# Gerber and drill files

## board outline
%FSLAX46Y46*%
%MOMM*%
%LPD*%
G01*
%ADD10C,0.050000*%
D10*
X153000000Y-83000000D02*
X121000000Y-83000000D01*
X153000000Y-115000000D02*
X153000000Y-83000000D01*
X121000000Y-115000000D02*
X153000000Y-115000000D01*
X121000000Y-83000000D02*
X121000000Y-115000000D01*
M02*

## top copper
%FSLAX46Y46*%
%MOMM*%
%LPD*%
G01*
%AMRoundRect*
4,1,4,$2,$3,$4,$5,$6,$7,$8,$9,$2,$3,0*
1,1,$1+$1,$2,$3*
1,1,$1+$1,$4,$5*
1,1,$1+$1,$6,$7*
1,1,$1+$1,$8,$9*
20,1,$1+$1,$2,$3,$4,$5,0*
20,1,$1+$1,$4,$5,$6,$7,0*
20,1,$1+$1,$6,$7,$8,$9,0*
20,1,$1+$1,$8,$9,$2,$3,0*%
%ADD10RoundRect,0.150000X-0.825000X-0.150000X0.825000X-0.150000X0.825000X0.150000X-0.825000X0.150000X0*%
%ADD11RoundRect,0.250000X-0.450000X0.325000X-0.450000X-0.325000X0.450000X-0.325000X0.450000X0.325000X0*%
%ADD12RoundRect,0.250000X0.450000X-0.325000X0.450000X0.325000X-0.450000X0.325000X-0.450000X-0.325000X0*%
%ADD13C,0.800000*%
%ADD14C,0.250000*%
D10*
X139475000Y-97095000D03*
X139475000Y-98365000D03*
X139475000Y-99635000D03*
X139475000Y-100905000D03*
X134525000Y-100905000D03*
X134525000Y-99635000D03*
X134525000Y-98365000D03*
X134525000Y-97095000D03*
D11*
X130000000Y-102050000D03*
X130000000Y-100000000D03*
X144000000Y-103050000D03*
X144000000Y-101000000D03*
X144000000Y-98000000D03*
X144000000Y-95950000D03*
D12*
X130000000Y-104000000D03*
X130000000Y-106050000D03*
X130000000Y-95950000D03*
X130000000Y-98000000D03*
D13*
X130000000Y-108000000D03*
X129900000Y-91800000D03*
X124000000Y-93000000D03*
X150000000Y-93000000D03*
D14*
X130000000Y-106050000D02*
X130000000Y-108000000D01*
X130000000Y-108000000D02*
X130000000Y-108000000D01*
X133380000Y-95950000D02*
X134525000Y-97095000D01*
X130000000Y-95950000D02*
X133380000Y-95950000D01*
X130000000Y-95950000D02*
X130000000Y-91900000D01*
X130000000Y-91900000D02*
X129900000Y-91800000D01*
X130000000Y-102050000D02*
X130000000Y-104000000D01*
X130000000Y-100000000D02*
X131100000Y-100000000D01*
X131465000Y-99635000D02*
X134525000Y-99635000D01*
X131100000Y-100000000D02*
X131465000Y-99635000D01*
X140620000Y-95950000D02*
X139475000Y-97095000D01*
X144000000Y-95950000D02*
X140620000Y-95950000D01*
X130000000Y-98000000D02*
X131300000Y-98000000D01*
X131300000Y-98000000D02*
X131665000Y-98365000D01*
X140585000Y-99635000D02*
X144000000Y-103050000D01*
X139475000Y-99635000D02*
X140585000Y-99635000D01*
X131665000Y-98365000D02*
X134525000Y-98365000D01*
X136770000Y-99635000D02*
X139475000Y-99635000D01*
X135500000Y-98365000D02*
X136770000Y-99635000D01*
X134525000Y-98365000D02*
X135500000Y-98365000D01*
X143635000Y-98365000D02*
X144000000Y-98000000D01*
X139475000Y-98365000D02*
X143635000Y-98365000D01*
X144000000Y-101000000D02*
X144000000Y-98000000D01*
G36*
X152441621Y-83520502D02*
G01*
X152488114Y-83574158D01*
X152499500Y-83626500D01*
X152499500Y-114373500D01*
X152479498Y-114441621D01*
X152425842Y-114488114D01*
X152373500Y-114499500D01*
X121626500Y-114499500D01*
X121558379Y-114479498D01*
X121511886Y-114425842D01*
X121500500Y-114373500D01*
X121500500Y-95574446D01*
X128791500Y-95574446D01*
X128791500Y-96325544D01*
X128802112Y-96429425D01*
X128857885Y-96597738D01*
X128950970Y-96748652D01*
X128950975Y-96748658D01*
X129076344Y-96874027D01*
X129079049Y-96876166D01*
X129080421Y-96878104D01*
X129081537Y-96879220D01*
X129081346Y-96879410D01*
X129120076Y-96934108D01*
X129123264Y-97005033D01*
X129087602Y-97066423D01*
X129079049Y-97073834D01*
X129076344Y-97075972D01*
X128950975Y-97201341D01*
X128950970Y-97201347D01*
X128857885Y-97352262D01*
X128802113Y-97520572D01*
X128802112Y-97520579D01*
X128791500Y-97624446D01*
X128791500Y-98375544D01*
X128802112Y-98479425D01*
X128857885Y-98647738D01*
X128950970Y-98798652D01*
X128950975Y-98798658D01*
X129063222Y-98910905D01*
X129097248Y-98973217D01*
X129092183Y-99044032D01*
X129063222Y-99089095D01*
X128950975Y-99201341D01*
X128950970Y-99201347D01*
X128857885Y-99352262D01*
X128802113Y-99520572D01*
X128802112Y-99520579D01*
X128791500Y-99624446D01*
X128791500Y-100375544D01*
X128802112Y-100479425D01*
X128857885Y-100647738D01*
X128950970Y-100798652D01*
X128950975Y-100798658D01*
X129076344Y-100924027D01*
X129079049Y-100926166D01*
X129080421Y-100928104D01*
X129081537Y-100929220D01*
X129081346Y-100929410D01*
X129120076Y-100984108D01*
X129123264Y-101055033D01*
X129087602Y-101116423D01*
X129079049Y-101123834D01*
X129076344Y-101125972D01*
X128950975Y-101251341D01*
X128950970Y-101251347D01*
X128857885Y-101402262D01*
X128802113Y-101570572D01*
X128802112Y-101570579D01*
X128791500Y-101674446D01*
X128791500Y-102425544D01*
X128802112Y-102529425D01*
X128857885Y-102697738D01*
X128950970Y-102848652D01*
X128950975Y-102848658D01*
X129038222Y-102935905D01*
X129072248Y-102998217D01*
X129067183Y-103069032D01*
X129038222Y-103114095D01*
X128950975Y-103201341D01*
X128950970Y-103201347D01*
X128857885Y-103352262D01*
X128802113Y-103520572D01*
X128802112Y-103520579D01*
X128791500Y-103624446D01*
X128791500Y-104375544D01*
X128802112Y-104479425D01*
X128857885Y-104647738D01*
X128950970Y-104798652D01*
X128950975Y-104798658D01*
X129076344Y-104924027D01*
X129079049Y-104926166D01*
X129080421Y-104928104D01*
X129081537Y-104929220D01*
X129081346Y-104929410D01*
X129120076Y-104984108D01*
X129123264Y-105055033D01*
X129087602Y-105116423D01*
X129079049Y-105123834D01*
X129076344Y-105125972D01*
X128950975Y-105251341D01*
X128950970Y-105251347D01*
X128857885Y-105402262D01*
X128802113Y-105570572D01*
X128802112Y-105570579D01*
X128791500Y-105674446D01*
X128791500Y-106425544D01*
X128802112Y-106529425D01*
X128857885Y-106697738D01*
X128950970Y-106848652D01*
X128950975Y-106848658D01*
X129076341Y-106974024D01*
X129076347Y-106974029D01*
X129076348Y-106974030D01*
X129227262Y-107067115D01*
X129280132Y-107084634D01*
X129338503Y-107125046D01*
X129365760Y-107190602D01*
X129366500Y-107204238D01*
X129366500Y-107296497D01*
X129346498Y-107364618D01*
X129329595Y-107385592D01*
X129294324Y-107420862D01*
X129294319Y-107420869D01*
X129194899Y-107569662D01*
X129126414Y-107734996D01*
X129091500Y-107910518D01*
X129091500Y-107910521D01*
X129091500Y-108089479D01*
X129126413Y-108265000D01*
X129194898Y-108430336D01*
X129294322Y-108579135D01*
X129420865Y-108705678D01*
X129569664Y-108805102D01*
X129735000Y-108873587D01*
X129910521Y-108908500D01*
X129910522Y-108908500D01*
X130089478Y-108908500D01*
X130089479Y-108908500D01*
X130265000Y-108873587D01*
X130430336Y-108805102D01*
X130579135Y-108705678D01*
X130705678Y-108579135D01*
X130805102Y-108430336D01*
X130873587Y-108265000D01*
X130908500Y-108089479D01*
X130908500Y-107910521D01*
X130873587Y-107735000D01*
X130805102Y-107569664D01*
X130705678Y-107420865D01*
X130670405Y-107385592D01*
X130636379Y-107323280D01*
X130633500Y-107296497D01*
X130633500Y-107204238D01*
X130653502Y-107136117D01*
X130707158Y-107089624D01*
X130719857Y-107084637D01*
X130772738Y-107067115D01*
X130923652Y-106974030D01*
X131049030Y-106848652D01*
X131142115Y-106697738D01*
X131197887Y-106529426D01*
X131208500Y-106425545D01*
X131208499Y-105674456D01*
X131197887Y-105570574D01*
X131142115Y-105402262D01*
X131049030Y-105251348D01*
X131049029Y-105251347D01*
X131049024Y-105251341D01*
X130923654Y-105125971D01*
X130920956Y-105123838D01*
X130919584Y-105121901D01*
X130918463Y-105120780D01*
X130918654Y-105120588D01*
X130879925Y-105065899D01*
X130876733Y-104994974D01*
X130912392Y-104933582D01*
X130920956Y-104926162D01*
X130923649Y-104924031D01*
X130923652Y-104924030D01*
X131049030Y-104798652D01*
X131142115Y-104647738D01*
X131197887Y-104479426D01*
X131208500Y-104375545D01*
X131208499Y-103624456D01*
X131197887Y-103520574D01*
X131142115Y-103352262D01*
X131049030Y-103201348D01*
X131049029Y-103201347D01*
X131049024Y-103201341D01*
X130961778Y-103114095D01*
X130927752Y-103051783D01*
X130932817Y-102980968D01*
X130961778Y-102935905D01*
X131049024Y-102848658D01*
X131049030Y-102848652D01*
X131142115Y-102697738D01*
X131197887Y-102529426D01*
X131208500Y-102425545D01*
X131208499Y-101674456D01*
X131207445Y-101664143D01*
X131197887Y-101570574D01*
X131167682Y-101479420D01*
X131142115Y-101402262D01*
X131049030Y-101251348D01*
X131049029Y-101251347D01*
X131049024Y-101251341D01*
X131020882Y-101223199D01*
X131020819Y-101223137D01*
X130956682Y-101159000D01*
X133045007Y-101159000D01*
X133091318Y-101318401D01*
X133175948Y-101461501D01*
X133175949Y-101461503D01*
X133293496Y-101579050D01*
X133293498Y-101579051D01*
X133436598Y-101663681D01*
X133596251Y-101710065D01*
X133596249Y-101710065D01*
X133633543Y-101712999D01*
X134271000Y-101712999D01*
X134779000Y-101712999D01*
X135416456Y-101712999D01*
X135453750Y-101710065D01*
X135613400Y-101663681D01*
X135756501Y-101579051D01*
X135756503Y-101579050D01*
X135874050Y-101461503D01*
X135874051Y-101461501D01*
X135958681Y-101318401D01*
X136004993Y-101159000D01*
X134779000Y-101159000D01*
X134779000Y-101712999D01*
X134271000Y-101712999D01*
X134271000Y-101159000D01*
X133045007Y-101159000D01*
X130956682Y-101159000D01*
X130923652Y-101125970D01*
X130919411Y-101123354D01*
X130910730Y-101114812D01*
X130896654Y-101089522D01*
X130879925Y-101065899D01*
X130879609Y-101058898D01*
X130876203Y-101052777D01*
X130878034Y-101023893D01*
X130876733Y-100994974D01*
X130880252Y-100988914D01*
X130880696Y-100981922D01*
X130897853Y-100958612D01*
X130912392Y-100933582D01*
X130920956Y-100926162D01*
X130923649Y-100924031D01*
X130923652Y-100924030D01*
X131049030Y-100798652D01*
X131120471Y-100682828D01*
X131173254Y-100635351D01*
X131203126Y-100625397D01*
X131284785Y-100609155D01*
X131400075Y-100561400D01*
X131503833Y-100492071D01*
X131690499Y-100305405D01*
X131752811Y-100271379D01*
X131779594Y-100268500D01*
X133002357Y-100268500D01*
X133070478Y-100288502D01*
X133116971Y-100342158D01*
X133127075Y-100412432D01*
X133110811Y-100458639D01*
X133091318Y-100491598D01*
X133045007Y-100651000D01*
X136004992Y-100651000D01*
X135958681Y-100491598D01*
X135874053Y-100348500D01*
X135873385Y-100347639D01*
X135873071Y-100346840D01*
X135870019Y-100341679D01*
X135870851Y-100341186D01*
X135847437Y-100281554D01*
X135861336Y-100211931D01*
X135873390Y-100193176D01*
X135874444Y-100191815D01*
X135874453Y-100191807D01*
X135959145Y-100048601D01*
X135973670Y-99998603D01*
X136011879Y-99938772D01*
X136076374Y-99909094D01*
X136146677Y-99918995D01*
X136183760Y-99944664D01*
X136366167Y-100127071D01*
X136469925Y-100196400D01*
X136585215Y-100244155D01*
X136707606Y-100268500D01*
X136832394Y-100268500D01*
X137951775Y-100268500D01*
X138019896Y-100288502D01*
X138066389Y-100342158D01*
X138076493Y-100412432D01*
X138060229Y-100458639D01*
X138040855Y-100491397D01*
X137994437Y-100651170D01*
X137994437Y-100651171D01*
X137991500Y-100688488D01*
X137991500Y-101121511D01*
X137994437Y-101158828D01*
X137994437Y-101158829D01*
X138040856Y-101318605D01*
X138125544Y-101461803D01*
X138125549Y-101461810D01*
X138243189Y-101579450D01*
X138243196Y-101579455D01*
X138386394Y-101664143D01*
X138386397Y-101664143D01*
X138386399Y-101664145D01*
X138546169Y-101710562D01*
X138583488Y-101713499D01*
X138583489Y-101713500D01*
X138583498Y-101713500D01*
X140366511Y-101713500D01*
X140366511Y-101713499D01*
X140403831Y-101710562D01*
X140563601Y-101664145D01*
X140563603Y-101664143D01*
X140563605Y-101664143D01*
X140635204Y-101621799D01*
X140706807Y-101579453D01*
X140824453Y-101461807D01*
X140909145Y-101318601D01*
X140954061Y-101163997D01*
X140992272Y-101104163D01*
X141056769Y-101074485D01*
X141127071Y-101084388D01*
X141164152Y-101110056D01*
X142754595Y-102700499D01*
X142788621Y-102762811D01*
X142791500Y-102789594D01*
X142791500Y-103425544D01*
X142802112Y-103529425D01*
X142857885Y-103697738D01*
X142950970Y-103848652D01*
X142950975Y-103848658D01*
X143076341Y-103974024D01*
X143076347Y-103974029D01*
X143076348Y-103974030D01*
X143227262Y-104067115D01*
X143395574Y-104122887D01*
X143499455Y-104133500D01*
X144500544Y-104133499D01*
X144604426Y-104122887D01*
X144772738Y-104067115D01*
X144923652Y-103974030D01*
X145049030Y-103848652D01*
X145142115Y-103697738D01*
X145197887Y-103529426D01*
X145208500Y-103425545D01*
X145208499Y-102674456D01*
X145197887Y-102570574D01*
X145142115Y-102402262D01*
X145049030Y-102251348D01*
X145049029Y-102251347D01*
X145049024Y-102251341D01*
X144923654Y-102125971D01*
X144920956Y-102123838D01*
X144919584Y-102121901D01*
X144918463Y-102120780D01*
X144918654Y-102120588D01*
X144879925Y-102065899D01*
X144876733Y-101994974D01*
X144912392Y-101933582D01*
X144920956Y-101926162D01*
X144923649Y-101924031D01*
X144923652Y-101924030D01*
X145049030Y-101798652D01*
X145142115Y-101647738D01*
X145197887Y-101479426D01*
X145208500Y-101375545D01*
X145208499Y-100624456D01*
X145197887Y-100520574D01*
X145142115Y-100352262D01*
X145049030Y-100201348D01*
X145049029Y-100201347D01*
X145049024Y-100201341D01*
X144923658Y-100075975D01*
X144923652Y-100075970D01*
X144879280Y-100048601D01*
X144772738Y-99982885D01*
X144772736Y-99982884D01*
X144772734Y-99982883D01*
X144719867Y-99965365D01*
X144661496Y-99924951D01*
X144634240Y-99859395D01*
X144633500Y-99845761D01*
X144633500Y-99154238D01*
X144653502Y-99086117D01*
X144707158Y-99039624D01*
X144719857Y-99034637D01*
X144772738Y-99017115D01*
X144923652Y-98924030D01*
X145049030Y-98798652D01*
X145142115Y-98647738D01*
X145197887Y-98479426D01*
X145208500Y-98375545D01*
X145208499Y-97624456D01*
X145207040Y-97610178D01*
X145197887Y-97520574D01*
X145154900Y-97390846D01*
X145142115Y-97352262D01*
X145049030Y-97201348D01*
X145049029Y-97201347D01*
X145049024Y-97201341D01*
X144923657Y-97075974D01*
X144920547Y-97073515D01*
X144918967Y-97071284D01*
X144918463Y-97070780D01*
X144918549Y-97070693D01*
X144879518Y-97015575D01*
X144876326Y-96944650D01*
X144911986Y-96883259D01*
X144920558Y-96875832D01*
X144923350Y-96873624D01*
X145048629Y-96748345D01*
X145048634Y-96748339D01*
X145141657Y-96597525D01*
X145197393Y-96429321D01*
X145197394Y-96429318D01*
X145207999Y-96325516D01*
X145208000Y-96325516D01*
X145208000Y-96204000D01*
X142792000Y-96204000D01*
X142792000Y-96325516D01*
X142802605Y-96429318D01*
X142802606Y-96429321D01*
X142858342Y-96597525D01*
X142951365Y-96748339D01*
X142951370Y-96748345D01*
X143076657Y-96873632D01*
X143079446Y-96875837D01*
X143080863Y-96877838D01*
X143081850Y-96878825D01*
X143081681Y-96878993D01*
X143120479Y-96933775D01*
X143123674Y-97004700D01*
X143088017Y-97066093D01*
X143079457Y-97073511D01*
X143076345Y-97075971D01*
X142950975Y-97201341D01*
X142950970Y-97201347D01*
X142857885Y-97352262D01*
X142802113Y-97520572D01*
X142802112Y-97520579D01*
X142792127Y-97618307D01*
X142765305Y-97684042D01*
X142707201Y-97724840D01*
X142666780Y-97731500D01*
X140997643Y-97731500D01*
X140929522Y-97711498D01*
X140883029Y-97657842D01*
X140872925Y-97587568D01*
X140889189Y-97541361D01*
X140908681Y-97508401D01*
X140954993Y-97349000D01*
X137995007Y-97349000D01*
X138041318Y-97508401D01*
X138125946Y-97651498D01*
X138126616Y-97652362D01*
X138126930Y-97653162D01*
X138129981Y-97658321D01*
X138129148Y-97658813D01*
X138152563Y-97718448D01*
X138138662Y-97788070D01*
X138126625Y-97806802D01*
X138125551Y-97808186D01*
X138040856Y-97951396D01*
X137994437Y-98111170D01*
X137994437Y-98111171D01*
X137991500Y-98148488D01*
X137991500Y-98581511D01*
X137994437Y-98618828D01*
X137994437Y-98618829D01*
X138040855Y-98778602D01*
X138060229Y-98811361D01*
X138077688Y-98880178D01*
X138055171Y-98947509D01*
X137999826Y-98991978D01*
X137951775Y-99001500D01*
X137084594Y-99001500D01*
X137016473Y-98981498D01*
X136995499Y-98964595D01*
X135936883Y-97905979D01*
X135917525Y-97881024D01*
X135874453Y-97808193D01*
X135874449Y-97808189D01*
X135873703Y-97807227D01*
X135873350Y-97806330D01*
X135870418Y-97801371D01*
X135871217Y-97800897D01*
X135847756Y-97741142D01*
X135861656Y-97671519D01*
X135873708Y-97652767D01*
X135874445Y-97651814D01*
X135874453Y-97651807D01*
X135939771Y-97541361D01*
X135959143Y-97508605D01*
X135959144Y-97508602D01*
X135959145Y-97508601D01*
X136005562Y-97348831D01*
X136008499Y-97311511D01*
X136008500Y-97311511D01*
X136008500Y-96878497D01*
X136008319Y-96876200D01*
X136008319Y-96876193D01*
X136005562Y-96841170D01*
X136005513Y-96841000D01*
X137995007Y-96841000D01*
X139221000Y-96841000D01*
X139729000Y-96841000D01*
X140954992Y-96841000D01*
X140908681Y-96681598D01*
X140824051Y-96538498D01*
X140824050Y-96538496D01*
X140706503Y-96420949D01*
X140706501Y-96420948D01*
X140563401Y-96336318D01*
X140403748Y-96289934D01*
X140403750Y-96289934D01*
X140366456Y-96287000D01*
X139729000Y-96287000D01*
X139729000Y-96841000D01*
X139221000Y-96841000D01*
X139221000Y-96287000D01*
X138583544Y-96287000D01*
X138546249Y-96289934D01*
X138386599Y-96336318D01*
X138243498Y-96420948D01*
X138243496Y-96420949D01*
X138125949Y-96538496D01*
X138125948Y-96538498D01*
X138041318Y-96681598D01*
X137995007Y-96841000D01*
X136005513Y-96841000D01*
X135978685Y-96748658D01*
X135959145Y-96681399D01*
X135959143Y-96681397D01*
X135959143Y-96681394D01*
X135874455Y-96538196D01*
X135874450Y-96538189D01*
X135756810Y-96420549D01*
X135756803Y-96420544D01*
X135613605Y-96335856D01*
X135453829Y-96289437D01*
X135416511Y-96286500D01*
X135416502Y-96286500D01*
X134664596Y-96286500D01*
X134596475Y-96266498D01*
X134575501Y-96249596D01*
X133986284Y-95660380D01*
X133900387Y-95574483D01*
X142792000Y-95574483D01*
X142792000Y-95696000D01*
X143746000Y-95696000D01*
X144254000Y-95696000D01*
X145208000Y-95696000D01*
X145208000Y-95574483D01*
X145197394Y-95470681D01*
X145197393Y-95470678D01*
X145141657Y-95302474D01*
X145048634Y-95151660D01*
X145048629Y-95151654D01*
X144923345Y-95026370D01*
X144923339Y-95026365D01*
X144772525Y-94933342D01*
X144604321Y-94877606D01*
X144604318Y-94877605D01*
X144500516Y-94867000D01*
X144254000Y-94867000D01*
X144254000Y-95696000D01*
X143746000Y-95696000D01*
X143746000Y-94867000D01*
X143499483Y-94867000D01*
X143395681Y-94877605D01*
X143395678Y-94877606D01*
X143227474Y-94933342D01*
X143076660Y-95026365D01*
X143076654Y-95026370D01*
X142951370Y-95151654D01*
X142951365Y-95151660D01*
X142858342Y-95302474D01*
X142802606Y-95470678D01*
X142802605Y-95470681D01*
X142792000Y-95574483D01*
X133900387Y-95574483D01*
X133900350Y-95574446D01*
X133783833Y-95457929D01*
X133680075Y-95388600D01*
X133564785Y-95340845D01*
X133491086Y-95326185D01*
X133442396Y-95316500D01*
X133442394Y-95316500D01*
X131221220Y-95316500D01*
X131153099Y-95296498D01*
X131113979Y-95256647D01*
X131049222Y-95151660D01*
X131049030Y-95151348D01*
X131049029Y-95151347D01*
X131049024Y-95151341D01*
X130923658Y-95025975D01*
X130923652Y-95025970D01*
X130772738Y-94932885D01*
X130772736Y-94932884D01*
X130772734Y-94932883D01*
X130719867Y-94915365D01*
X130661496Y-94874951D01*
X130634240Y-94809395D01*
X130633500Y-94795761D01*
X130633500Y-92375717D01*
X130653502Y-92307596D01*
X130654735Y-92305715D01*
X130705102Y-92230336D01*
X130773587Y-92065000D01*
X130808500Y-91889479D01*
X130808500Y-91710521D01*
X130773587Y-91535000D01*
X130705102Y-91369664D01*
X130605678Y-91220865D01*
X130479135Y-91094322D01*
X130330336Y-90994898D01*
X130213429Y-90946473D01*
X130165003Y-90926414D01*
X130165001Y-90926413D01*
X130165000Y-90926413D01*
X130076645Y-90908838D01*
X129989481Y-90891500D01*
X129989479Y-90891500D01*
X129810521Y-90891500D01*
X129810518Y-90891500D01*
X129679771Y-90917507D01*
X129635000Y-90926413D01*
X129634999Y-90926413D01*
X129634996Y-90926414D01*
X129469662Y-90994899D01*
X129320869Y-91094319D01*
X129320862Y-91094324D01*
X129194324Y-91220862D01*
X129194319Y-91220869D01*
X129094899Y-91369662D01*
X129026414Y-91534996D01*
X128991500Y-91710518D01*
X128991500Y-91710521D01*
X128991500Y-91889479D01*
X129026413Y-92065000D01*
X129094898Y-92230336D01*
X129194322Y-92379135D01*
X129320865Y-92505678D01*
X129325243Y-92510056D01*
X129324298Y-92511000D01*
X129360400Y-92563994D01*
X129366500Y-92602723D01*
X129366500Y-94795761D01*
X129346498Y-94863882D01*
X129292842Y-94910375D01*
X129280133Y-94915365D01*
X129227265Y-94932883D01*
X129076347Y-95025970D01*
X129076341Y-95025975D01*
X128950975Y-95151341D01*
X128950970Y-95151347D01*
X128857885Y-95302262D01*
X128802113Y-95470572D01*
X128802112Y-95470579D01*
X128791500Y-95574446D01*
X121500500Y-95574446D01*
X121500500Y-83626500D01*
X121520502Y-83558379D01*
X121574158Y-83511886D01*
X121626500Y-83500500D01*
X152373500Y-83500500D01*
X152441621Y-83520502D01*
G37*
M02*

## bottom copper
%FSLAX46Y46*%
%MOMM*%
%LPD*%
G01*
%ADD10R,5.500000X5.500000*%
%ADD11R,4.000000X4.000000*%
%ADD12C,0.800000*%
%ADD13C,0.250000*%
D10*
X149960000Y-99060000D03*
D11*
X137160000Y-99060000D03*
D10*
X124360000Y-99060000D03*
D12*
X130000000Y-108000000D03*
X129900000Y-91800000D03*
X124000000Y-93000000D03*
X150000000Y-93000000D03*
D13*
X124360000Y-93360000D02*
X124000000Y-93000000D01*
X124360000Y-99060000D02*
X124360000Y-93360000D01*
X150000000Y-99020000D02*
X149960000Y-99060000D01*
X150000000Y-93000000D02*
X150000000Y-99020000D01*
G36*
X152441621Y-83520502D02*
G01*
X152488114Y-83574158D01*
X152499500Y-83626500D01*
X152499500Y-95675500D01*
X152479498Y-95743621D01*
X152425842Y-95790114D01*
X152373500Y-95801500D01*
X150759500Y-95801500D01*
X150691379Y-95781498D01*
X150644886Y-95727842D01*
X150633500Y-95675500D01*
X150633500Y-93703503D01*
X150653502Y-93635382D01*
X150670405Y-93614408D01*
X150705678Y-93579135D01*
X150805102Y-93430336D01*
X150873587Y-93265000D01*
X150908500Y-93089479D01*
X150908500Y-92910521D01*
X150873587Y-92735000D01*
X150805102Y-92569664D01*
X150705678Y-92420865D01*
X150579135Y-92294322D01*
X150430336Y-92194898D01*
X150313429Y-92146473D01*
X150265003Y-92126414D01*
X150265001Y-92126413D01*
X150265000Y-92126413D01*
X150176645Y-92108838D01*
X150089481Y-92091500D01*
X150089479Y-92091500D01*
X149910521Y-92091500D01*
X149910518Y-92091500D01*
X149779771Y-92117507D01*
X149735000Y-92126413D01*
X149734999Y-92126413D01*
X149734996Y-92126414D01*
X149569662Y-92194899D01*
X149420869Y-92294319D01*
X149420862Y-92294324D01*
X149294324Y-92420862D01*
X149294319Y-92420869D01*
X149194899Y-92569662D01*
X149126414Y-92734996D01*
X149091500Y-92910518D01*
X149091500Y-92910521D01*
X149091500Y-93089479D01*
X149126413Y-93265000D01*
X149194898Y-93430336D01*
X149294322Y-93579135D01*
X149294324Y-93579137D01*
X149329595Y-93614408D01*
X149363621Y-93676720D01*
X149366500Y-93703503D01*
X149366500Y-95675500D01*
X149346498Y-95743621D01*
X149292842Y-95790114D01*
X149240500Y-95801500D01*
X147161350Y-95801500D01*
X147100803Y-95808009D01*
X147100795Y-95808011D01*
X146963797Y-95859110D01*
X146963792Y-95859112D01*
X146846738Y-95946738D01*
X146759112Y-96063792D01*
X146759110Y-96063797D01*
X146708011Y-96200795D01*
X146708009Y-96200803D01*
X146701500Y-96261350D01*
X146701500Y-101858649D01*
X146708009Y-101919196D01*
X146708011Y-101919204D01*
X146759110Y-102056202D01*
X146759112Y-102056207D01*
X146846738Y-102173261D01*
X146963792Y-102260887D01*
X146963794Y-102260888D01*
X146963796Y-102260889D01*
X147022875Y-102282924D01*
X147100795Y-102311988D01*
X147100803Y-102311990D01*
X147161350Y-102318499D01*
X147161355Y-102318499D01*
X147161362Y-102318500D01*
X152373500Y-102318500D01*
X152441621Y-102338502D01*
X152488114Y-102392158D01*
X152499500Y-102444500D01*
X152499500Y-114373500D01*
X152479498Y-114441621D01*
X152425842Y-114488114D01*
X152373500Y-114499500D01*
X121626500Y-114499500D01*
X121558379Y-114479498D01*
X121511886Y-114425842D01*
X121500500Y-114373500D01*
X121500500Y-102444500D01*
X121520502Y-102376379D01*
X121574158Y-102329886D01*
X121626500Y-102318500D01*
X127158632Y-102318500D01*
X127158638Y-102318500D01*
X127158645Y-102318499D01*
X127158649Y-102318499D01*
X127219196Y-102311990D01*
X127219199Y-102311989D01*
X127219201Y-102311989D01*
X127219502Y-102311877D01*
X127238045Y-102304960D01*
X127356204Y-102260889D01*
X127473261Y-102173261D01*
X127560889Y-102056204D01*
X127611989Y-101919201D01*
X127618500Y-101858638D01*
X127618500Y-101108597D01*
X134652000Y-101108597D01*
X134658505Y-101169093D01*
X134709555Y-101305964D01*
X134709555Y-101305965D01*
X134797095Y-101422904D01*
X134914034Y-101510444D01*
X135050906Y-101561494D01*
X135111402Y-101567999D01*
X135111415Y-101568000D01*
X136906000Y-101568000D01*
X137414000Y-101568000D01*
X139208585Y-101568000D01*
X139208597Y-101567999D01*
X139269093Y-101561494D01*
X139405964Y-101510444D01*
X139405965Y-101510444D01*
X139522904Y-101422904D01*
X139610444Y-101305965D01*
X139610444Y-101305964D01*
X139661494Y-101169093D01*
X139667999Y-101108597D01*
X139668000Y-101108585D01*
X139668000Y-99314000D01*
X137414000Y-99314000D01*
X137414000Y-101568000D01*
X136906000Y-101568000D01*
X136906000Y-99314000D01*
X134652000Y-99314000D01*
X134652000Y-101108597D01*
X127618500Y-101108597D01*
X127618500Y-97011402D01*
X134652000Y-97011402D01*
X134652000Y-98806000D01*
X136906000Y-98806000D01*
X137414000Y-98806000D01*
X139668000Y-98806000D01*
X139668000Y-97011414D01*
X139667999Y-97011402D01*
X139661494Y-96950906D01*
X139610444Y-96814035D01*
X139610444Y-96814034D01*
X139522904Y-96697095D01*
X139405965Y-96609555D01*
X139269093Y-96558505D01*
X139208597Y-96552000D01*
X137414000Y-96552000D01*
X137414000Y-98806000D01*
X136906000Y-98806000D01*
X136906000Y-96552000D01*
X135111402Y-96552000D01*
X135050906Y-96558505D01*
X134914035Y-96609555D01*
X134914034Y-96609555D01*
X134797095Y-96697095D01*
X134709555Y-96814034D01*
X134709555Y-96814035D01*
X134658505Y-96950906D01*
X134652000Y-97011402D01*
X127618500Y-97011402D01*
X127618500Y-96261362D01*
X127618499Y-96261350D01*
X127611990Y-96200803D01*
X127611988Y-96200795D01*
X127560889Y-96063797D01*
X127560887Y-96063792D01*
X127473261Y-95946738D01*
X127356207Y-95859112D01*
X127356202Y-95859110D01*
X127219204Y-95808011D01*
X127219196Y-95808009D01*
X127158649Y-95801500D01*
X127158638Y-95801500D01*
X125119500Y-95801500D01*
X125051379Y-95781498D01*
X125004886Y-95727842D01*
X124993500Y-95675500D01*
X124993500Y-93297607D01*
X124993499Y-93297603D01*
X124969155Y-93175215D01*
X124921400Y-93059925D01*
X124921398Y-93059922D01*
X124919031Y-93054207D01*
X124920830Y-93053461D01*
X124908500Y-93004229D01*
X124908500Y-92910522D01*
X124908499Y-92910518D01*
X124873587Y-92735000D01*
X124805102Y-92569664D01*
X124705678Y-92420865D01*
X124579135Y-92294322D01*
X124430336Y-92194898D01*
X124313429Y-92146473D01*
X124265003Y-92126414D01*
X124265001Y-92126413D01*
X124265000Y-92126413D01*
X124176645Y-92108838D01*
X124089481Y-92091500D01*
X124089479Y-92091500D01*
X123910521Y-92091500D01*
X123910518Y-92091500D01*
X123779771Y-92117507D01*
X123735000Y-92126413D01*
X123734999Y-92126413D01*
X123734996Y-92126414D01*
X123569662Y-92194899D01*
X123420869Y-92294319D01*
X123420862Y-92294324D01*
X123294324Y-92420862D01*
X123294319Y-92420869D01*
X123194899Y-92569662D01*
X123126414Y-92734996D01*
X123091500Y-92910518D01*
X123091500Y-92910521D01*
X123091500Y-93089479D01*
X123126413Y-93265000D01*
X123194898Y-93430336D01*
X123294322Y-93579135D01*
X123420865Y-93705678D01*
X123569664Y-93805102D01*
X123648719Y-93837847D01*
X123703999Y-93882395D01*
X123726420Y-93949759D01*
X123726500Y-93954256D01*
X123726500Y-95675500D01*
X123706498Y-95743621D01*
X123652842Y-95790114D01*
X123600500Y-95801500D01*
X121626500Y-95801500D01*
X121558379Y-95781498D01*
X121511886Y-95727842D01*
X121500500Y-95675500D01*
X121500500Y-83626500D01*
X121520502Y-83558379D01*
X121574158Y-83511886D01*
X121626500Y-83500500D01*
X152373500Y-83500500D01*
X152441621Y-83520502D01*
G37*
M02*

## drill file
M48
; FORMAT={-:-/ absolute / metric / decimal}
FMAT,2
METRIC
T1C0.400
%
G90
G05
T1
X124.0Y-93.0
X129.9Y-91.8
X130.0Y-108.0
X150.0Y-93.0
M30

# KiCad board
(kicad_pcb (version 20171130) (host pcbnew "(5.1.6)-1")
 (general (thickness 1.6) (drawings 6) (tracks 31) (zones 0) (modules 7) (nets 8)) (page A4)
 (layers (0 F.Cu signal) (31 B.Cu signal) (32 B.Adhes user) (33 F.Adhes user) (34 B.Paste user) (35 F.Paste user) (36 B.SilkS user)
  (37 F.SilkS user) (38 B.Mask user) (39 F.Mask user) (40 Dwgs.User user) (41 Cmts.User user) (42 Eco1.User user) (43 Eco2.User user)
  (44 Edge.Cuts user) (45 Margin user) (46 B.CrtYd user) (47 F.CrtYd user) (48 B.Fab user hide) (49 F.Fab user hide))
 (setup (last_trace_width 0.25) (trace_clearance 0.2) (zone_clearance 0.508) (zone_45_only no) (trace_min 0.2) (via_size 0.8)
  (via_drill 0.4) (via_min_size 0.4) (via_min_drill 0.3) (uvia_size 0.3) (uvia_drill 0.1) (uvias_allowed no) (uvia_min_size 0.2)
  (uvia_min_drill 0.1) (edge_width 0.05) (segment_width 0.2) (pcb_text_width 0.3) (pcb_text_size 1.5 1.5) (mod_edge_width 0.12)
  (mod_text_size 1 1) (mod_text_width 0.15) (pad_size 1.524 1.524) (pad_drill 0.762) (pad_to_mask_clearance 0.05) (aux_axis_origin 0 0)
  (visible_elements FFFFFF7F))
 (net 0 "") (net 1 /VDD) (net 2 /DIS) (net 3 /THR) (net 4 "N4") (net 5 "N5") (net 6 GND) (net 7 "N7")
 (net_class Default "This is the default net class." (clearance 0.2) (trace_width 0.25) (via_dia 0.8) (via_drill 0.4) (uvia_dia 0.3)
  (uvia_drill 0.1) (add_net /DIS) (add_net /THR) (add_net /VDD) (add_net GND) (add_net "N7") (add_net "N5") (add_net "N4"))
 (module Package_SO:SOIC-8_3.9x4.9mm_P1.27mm (layer F.Cu) (at 137 99)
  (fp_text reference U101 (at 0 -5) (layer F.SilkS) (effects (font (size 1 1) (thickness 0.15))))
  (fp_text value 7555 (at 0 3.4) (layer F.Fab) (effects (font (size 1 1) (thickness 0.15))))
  (pad 8 smd roundrect (at 2.475 -1.905) (size 1.95 0.6) (layers F.Cu F.Paste F.Mask) (roundrect_rratio 0.25) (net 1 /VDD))
  (pad 7 smd roundrect (at 2.475 -0.635) (size 1.95 0.6) (layers F.Cu F.Paste F.Mask) (roundrect_rratio 0.25) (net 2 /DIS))
  (pad 6 smd roundrect (at 2.475 0.635) (size 1.95 0.6) (layers F.Cu F.Paste F.Mask) (roundrect_rratio 0.25) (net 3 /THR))
  (pad 5 smd roundrect (at 2.475 1.905) (size 1.95 0.6) (layers F.Cu F.Paste F.Mask) (roundrect_rratio 0.25) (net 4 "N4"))
  (pad 4 smd roundrect (at -2.475 1.905) (size 1.95 0.6) (layers F.Cu F.Paste F.Mask) (roundrect_rratio 0.25) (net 1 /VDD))
  (pad 3 smd roundrect (at -2.475 0.635) (size 1.95 0.6) (layers F.Cu F.Paste F.Mask) (roundrect_rratio 0.25) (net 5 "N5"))
  (pad 2 smd roundrect (at -2.475 -0.635) (size 1.95 0.6) (layers F.Cu F.Paste F.Mask) (roundrect_rratio 0.25) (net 3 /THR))
  (pad 1 smd roundrect (at -2.475 -1.905) (size 1.95 0.6) (layers F.Cu F.Paste F.Mask) (roundrect_rratio 0.25) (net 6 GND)))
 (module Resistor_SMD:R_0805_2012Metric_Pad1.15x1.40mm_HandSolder (layer F.Cu) (at 130 101.025 270)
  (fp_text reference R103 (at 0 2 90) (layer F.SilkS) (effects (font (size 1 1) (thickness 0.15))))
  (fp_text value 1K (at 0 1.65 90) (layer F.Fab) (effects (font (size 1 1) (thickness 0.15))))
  (pad 2 smd roundrect (at 1.025 0 270) (size 1.15 1.4) (layers F.Cu F.Paste F.Mask) (roundrect_rratio 0.217391) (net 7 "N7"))
  (pad 1 smd roundrect (at -1.025 0 270) (size 1.15 1.4) (layers F.Cu F.Paste F.Mask) (roundrect_rratio 0.217391) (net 5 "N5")))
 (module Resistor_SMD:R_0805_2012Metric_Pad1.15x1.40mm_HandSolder (layer F.Cu) (at 144 102.025 270)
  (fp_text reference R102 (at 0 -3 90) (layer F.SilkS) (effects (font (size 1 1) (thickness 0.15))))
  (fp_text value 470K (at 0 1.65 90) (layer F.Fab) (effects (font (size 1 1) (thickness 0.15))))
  (pad 2 smd roundrect (at 1.025 0 270) (size 1.15 1.4) (layers F.Cu F.Paste F.Mask) (roundrect_rratio 0.217391) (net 3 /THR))
  (pad 1 smd roundrect (at -1.025 0 270) (size 1.15 1.4) (layers F.Cu F.Paste F.Mask) (roundrect_rratio 0.217391) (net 2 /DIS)))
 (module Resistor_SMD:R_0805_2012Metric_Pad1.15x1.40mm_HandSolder (layer F.Cu) (at 144 96.975 270)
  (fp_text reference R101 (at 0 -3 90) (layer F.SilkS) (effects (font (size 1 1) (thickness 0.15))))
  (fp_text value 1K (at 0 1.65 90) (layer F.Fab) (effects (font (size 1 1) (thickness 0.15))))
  (pad 2 smd roundrect (at 1.025 0 270) (size 1.15 1.4) (layers F.Cu F.Paste F.Mask) (roundrect_rratio 0.217391) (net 2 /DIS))
  (pad 1 smd roundrect (at -1.025 0 270) (size 1.15 1.4) (layers F.Cu F.Paste F.Mask) (roundrect_rratio 0.217391) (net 1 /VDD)))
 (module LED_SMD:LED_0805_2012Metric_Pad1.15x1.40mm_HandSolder (layer F.Cu) (at 130 105.025 90)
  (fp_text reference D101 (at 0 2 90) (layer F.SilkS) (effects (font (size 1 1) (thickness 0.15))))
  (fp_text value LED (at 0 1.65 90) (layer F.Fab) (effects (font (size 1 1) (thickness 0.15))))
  (pad 2 smd roundrect (at 1.025 0 90) (size 1.15 1.4) (layers F.Cu F.Paste F.Mask) (roundrect_rratio 0.217391) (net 7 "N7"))
  (pad 1 smd roundrect (at -1.025 0 90) (size 1.15 1.4) (layers F.Cu F.Paste F.Mask) (roundrect_rratio 0.217391) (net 6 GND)))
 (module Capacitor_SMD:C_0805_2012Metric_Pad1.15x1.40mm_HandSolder (layer F.Cu) (at 130 96.975 90)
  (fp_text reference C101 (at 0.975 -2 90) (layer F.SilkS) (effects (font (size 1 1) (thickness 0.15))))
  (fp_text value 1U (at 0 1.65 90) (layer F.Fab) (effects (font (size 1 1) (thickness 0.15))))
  (pad 2 smd roundrect (at 1.025 0 90) (size 1.15 1.4) (layers F.Cu F.Paste F.Mask) (roundrect_rratio 0.217391) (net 6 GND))
  (pad 1 smd roundrect (at -1.025 0 90) (size 1.15 1.4) (layers F.Cu F.Paste F.Mask) (roundrect_rratio 0.217391) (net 3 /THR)))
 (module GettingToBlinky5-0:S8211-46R (layer B.Cu) (at 137.16 99.06)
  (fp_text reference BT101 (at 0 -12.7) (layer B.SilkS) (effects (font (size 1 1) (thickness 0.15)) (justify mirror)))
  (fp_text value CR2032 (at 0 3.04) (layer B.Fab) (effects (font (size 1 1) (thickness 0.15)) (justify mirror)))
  (pad 1 smd rect (at 12.8 0) (size 5.5 5.5) (layers B.Cu B.Paste B.Mask) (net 1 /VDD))
  (pad 2 smd rect (at 0 0) (size 4 4) (layers B.Cu B.Paste B.Mask) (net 6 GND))
  (pad 1 smd rect (at -12.8 0) (size 5.5 5.5) (layers B.Cu B.Paste B.Mask) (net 1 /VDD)))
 (gr_line (start 153 83) (end 121 83) (layer Edge.Cuts) (width 0.05))
 (gr_line (start 153 115) (end 153 83) (layer Edge.Cuts) (width 0.05))
 (gr_line (start 121 115) (end 153 115) (layer Edge.Cuts) (width 0.05))
 (gr_line (start 121 83) (end 121 115) (layer Edge.Cuts) (width 0.05))
 (segment (start 130 106.05) (end 130 108) (width 0.25) (layer F.Cu) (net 6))
 (segment (start 130 108) (end 130 108) (width 0.25) (layer F.Cu) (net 6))
 (via (at 130 108) (size 0.8) (drill 0.4) (layers F.Cu B.Cu) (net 6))
 (segment (start 133.38 95.95) (end 134.525 97.095) (width 0.25) (layer F.Cu) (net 6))
 (segment (start 130 95.95) (end 133.38 95.95) (width 0.25) (layer F.Cu) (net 6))
 (via (at 129.9 91.8) (size 0.8) (drill 0.4) (layers F.Cu B.Cu) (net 6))
 (segment (start 130 95.95) (end 130 91.9) (width 0.25) (layer F.Cu) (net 6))
 (segment (start 130 91.9) (end 129.9 91.8) (width 0.25) (layer F.Cu) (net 6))
 (segment (start 130 102.05) (end 130 104) (width 0.25) (layer F.Cu) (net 7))
 (segment (start 130 100) (end 131.1 100) (width 0.25) (layer F.Cu) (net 5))
 (segment (start 131.465 99.635) (end 134.525 99.635) (width 0.25) (layer F.Cu) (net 5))
 (segment (start 131.1 100) (end 131.465 99.635) (width 0.25) (layer F.Cu) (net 5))
 (segment (start 140.62 95.95) (end 139.475 97.095) (width 0.25) (layer F.Cu) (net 1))
 (segment (start 144 95.95) (end 140.62 95.95) (width 0.25) (layer F.Cu) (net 1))
 (via (at 124 93) (size 0.8) (drill 0.4) (layers F.Cu B.Cu) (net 1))
 (segment (start 124.36 93.36) (end 124 93) (width 0.25) (layer B.Cu) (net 1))
 (segment (start 124.36 99.06) (end 124.36 93.36) (width 0.25) (layer B.Cu) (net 1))
 (via (at 150 93) (size 0.8) (drill 0.4) (layers F.Cu B.Cu) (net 1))
 (segment (start 150 99.02) (end 149.96 99.06) (width 0.25) (layer B.Cu) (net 1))
 (segment (start 150 93) (end 150 99.02) (width 0.25) (layer B.Cu) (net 1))
 (segment (start 130 98) (end 131.3 98) (width 0.25) (layer F.Cu) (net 3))
 (segment (start 131.3 98) (end 131.665 98.365) (width 0.25) (layer F.Cu) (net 3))
 (segment (start 140.585 99.635) (end 144 103.05) (width 0.25) (layer F.Cu) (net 3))
 (segment (start 139.475 99.635) (end 140.585 99.635) (width 0.25) (layer F.Cu) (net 3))
 (segment (start 131.665 98.365) (end 134.525 98.365) (width 0.25) (layer F.Cu) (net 3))
 (segment (start 136.77 99.635) (end 139.475 99.635) (width 0.25) (layer F.Cu) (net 3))
 (segment (start 135.5 98.365) (end 136.77 99.635) (width 0.25) (layer F.Cu) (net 3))
 (segment (start 134.525 98.365) (end 135.5 98.365) (width 0.25) (layer F.Cu) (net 3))
 (segment (start 143.635 98.365) (end 144 98) (width 0.25) (layer F.Cu) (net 2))
 (segment (start 139.475 98.365) (end 143.635 98.365) (width 0.25) (layer F.Cu) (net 2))
 (segment (start 144 101) (end 144 98) (width 0.25) (layer F.Cu) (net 2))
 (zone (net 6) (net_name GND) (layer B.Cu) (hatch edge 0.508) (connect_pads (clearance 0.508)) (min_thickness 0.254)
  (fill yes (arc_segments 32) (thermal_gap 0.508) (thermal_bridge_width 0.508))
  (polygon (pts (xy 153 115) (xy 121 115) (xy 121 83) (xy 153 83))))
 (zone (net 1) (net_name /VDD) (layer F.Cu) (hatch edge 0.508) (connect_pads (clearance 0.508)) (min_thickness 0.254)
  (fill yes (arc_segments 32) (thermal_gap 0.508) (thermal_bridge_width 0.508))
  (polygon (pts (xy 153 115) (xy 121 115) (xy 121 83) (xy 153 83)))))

